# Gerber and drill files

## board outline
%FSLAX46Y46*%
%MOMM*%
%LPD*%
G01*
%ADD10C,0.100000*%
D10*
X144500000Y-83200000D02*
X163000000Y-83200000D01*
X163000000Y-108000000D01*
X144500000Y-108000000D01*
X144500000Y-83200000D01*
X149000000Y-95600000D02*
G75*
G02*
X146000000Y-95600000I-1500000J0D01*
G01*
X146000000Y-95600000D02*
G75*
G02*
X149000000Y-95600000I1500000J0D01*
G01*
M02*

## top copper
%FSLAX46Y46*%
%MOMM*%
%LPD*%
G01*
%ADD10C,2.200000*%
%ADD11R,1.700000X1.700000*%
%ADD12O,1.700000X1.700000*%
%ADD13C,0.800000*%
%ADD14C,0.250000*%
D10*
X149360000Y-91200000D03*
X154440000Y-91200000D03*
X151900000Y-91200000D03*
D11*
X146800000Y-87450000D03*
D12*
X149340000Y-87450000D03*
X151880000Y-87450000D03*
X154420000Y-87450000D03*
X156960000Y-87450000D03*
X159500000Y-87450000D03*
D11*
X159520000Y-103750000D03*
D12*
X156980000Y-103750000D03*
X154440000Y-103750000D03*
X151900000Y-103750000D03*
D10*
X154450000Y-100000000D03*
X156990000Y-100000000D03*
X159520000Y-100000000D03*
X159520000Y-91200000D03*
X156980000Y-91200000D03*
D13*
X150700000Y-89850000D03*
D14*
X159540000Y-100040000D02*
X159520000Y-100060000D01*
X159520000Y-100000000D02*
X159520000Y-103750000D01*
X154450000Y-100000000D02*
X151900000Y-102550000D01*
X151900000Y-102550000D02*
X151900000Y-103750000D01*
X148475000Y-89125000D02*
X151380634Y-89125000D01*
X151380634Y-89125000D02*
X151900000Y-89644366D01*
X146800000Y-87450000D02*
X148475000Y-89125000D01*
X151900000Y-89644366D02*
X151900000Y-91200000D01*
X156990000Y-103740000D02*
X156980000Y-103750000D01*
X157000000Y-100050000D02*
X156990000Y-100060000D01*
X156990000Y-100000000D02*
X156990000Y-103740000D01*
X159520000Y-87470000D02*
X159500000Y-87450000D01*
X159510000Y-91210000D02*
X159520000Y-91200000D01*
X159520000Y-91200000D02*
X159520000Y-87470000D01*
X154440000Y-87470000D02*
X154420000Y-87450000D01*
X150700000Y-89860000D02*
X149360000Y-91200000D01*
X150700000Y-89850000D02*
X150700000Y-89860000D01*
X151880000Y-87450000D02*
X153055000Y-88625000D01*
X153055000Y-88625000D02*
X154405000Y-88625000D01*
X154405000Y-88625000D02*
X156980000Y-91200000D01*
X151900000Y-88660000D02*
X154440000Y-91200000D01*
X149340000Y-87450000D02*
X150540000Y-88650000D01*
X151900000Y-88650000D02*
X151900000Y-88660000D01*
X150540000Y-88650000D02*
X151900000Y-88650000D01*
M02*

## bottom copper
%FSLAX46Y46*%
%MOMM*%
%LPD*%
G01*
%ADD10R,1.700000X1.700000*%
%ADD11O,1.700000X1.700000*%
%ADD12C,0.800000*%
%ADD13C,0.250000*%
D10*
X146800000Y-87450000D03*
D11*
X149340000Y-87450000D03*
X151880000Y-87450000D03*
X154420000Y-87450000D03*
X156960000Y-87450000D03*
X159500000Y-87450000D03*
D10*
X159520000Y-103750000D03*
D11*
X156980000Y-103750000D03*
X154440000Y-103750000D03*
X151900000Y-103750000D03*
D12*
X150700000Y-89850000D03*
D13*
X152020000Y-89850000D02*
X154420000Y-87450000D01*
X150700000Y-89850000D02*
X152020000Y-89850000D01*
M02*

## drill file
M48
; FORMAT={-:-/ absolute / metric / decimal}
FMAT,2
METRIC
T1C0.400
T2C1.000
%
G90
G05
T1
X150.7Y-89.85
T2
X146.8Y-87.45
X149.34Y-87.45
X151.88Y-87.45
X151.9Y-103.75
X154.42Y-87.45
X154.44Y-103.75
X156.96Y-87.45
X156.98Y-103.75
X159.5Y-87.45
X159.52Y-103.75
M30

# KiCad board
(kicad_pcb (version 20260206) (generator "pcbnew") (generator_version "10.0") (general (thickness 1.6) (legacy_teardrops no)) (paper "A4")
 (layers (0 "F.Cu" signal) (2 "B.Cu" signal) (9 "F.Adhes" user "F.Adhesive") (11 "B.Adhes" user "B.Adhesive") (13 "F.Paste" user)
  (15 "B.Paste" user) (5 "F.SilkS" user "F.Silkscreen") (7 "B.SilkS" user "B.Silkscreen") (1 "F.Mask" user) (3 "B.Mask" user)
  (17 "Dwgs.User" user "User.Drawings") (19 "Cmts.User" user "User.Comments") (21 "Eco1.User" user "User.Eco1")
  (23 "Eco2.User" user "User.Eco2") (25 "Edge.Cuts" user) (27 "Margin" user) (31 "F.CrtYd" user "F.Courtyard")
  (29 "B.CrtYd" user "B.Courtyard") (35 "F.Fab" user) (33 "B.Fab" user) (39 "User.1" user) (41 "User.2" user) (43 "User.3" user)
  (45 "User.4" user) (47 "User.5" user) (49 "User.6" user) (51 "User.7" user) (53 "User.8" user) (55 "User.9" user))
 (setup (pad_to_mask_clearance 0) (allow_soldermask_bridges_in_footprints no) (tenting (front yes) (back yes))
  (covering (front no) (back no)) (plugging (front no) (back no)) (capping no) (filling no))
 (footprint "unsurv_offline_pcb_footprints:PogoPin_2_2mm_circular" (layer "F.Cu") (at 149.36 91.2)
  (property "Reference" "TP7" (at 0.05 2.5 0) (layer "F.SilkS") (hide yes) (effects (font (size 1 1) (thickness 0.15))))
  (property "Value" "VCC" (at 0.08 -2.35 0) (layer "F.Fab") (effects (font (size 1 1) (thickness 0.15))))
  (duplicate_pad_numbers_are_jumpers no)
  (pad "1" smd circle (at 0 0) (size 2.2 2.2) (layers "F.Cu" "F.Mask" "F.Paste") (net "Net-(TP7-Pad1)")))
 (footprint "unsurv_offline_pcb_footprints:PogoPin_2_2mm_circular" (layer "F.Cu") (at 154.44 91.2)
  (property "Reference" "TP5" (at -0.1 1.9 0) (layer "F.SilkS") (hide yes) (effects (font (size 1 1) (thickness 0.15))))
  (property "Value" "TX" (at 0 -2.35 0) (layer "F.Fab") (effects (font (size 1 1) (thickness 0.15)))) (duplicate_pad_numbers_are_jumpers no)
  (pad "1" smd circle (at 0 0) (size 2.2 2.2) (layers "F.Cu" "F.Mask" "F.Paste") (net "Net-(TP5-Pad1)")))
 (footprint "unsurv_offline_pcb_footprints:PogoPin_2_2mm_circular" (layer "F.Cu") (at 151.9 91.2)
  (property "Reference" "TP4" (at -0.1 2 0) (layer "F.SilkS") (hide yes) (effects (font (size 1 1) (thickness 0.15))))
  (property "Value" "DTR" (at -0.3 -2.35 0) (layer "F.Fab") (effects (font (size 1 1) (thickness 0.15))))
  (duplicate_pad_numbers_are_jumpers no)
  (pad "1" smd circle (at 0 0) (size 2.2 2.2) (layers "F.Cu" "F.Mask" "F.Paste") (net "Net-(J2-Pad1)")))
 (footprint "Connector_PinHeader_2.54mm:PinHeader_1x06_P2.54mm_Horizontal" (layer "F.Cu") (at 146.8 87.45 90)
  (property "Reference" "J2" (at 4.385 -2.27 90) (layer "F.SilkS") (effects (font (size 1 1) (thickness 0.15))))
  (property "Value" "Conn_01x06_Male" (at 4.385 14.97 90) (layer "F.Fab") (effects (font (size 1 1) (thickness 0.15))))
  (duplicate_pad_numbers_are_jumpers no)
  (pad "1" thru_hole rect (at 0 0 90) (size 1.7 1.7) (drill 1) (layers "*.Cu" "*.Mask") (remove_unused_layers no) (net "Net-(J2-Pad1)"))
  (pad "2" thru_hole oval (at 0 2.54 90) (size 1.7 1.7) (drill 1) (layers "*.Cu" "*.Mask") (remove_unused_layers no) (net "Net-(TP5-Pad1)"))
  (pad "3" thru_hole oval (at 0 5.08 90) (size 1.7 1.7) (drill 1) (layers "*.Cu" "*.Mask") (remove_unused_layers no) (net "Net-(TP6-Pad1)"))
  (pad "4" thru_hole oval (at 0 7.62 90) (size 1.7 1.7) (drill 1) (layers "*.Cu" "*.Mask") (remove_unused_layers no) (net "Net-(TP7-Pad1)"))
  (pad "5" thru_hole oval (at 0 10.16 90) (size 1.7 1.7) (drill 1) (layers "*.Cu" "*.Mask") (remove_unused_layers no)
   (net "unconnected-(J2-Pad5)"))
  (pad "6" thru_hole oval (at 0 12.7 90) (size 1.7 1.7) (drill 1) (layers "*.Cu" "*.Mask") (remove_unused_layers no) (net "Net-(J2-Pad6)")))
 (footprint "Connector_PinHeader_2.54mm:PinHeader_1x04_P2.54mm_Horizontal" (layer "F.Cu") (at 159.52 103.75 -90)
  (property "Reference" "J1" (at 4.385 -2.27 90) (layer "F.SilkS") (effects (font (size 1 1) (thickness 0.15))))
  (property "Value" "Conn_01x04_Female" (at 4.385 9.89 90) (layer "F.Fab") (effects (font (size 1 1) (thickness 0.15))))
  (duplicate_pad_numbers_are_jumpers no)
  (pad "1" thru_hole rect (at 0 0 270) (size 1.7 1.7) (drill 1) (layers "*.Cu" "*.Mask") (remove_unused_layers no) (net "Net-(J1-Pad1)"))
  (pad "2" thru_hole oval (at 0 2.54 270) (size 1.7 1.7) (drill 1) (layers "*.Cu" "*.Mask") (remove_unused_layers no) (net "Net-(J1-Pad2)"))
  (pad "3" thru_hole oval (at 0 5.08 270) (size 1.7 1.7) (drill 1) (layers "*.Cu" "*.Mask") (remove_unused_layers no)
   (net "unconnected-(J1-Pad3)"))
  (pad "4" thru_hole oval (at 0 7.62 270) (size 1.7 1.7) (drill 1) (layers "*.Cu" "*.Mask") (remove_unused_layers no) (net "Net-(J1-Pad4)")))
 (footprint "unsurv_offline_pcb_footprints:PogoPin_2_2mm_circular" (layer "F.Cu") (at 154.45 100)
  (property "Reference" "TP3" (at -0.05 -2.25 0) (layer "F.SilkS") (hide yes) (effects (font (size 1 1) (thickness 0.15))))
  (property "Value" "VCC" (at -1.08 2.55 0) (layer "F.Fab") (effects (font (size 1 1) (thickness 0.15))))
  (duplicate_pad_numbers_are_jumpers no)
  (pad "1" smd circle (at 0 0) (size 2.2 2.2) (layers "F.Cu" "F.Mask" "F.Paste") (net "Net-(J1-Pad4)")))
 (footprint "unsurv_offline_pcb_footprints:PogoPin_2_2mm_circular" (layer "F.Cu") (at 156.99 100)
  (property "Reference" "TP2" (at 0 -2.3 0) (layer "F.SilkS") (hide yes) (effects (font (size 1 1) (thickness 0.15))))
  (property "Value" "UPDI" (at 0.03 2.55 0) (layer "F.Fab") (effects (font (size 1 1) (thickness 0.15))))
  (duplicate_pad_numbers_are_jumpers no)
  (pad "1" smd circle (at 0 0) (size 2.2 2.2) (layers "F.Cu" "F.Mask" "F.Paste") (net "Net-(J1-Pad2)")))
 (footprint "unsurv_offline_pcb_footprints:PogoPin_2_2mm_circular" (layer "F.Cu") (at 159.52 100)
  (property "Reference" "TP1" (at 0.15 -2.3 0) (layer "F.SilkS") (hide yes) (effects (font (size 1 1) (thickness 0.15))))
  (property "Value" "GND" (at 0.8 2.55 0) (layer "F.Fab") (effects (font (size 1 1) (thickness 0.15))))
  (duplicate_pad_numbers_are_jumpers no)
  (pad "1" smd circle (at 0 0) (size 2.2 2.2) (layers "F.Cu" "F.Mask" "F.Paste") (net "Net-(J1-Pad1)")))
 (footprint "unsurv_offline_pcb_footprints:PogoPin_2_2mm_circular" (layer "F.Cu") (at 159.52 91.2)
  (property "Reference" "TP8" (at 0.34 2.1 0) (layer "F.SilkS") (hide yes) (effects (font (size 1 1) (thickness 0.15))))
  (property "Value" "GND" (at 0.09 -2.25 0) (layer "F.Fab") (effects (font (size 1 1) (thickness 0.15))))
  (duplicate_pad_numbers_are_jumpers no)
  (pad "1" smd circle (at 0 0) (size 2.2 2.2) (layers "F.Cu" "F.Mask" "F.Paste") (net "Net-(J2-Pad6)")))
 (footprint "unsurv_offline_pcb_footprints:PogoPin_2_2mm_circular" (layer "F.Cu") (at 156.98 91.2)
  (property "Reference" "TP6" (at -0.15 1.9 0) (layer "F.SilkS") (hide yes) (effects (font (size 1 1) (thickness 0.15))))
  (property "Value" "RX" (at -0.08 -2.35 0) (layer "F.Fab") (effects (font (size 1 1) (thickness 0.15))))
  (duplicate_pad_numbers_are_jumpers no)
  (pad "1" smd circle (at 0 0) (size 2.2 2.2) (layers "F.Cu" "F.Mask" "F.Paste") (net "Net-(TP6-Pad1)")))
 (gr_rect (start 144.5 83.2) (end 163 108) (stroke (width 0.1) (type solid)) (fill no) (layer "Edge.Cuts"))
 (gr_circle (center 147.5 95.6) (end 149 95.6) (stroke (width 0.1) (type solid)) (fill no) (layer "Edge.Cuts"))
 (segment (start 159.54 100.04) (end 159.52 100.06) (width 0.25) (layer "F.Cu") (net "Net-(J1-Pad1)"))
 (segment (start 159.52 100) (end 159.52 103.75) (width 0.25) (layer "F.Cu") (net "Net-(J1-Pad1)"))
 (segment (start 154.45 100) (end 151.9 102.55) (width 0.25) (layer "F.Cu") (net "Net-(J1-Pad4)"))
 (segment (start 151.9 102.55) (end 151.9 103.75) (width 0.25) (layer "F.Cu") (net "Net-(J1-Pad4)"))
 (segment (start 148.475 89.125) (end 151.380634 89.125) (width 0.25) (layer "F.Cu") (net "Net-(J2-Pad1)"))
 (segment (start 151.380634 89.125) (end 151.9 89.644366) (width 0.25) (layer "F.Cu") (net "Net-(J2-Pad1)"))
 (segment (start 146.8 87.45) (end 148.475 89.125) (width 0.25) (layer "F.Cu") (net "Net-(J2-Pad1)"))
 (segment (start 151.9 89.644366) (end 151.9 91.2) (width 0.25) (layer "F.Cu") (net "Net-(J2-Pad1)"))
 (segment (start 156.99 103.74) (end 156.98 103.75) (width 0.25) (layer "F.Cu") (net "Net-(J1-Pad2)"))
 (segment (start 157 100.05) (end 156.99 100.06) (width 0.25) (layer "F.Cu") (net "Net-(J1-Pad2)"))
 (segment (start 156.99 100) (end 156.99 103.74) (width 0.25) (layer "F.Cu") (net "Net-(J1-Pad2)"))
 (segment (start 159.52 87.47) (end 159.5 87.45) (width 0.25) (layer "F.Cu") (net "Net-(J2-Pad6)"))
 (segment (start 159.51 91.21) (end 159.52 91.2) (width 0.25) (layer "F.Cu") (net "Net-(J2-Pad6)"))
 (segment (start 159.52 91.2) (end 159.52 87.47) (width 0.25) (layer "F.Cu") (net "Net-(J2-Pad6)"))
 (segment (start 154.44 87.47) (end 154.42 87.45) (width 0.25) (layer "F.Cu") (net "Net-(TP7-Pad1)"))
 (segment (start 150.7 89.86) (end 149.36 91.2) (width 0.25) (layer "F.Cu") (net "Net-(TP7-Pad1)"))
 (segment (start 150.7 89.85) (end 150.7 89.86) (width 0.25) (layer "F.Cu") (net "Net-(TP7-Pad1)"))
 (via (at 150.7 89.85) (size 0.8) (drill 0.4) (layers "F.Cu" "B.Cu") (capping no) (covering (front no) (back no))
  (plugging (front no) (back no)) (filling no) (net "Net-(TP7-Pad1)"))
 (segment (start 152.02 89.85) (end 154.42 87.45) (width 0.25) (layer "B.Cu") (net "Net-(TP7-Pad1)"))
 (segment (start 150.7 89.85) (end 152.02 89.85) (width 0.25) (layer "B.Cu") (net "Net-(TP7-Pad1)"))
 (segment (start 151.88 87.45) (end 153.055 88.625) (width 0.25) (layer "F.Cu") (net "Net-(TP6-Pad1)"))
 (segment (start 153.055 88.625) (end 154.405 88.625) (width 0.25) (layer "F.Cu") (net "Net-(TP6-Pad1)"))
 (segment (start 154.405 88.625) (end 156.98 91.2) (width 0.25) (layer "F.Cu") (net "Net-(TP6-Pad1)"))
 (segment (start 151.9 88.66) (end 154.44 91.2) (width 0.25) (layer "F.Cu") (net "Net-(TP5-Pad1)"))
 (segment (start 149.34 87.45) (end 150.54 88.65) (width 0.25) (layer "F.Cu") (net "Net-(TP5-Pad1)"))
 (segment (start 151.9 88.65) (end 151.9 88.66) (width 0.25) (layer "F.Cu") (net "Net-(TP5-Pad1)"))
 (segment (start 150.54 88.65) (end 151.9 88.65) (width 0.25) (layer "F.Cu") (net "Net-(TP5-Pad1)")))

